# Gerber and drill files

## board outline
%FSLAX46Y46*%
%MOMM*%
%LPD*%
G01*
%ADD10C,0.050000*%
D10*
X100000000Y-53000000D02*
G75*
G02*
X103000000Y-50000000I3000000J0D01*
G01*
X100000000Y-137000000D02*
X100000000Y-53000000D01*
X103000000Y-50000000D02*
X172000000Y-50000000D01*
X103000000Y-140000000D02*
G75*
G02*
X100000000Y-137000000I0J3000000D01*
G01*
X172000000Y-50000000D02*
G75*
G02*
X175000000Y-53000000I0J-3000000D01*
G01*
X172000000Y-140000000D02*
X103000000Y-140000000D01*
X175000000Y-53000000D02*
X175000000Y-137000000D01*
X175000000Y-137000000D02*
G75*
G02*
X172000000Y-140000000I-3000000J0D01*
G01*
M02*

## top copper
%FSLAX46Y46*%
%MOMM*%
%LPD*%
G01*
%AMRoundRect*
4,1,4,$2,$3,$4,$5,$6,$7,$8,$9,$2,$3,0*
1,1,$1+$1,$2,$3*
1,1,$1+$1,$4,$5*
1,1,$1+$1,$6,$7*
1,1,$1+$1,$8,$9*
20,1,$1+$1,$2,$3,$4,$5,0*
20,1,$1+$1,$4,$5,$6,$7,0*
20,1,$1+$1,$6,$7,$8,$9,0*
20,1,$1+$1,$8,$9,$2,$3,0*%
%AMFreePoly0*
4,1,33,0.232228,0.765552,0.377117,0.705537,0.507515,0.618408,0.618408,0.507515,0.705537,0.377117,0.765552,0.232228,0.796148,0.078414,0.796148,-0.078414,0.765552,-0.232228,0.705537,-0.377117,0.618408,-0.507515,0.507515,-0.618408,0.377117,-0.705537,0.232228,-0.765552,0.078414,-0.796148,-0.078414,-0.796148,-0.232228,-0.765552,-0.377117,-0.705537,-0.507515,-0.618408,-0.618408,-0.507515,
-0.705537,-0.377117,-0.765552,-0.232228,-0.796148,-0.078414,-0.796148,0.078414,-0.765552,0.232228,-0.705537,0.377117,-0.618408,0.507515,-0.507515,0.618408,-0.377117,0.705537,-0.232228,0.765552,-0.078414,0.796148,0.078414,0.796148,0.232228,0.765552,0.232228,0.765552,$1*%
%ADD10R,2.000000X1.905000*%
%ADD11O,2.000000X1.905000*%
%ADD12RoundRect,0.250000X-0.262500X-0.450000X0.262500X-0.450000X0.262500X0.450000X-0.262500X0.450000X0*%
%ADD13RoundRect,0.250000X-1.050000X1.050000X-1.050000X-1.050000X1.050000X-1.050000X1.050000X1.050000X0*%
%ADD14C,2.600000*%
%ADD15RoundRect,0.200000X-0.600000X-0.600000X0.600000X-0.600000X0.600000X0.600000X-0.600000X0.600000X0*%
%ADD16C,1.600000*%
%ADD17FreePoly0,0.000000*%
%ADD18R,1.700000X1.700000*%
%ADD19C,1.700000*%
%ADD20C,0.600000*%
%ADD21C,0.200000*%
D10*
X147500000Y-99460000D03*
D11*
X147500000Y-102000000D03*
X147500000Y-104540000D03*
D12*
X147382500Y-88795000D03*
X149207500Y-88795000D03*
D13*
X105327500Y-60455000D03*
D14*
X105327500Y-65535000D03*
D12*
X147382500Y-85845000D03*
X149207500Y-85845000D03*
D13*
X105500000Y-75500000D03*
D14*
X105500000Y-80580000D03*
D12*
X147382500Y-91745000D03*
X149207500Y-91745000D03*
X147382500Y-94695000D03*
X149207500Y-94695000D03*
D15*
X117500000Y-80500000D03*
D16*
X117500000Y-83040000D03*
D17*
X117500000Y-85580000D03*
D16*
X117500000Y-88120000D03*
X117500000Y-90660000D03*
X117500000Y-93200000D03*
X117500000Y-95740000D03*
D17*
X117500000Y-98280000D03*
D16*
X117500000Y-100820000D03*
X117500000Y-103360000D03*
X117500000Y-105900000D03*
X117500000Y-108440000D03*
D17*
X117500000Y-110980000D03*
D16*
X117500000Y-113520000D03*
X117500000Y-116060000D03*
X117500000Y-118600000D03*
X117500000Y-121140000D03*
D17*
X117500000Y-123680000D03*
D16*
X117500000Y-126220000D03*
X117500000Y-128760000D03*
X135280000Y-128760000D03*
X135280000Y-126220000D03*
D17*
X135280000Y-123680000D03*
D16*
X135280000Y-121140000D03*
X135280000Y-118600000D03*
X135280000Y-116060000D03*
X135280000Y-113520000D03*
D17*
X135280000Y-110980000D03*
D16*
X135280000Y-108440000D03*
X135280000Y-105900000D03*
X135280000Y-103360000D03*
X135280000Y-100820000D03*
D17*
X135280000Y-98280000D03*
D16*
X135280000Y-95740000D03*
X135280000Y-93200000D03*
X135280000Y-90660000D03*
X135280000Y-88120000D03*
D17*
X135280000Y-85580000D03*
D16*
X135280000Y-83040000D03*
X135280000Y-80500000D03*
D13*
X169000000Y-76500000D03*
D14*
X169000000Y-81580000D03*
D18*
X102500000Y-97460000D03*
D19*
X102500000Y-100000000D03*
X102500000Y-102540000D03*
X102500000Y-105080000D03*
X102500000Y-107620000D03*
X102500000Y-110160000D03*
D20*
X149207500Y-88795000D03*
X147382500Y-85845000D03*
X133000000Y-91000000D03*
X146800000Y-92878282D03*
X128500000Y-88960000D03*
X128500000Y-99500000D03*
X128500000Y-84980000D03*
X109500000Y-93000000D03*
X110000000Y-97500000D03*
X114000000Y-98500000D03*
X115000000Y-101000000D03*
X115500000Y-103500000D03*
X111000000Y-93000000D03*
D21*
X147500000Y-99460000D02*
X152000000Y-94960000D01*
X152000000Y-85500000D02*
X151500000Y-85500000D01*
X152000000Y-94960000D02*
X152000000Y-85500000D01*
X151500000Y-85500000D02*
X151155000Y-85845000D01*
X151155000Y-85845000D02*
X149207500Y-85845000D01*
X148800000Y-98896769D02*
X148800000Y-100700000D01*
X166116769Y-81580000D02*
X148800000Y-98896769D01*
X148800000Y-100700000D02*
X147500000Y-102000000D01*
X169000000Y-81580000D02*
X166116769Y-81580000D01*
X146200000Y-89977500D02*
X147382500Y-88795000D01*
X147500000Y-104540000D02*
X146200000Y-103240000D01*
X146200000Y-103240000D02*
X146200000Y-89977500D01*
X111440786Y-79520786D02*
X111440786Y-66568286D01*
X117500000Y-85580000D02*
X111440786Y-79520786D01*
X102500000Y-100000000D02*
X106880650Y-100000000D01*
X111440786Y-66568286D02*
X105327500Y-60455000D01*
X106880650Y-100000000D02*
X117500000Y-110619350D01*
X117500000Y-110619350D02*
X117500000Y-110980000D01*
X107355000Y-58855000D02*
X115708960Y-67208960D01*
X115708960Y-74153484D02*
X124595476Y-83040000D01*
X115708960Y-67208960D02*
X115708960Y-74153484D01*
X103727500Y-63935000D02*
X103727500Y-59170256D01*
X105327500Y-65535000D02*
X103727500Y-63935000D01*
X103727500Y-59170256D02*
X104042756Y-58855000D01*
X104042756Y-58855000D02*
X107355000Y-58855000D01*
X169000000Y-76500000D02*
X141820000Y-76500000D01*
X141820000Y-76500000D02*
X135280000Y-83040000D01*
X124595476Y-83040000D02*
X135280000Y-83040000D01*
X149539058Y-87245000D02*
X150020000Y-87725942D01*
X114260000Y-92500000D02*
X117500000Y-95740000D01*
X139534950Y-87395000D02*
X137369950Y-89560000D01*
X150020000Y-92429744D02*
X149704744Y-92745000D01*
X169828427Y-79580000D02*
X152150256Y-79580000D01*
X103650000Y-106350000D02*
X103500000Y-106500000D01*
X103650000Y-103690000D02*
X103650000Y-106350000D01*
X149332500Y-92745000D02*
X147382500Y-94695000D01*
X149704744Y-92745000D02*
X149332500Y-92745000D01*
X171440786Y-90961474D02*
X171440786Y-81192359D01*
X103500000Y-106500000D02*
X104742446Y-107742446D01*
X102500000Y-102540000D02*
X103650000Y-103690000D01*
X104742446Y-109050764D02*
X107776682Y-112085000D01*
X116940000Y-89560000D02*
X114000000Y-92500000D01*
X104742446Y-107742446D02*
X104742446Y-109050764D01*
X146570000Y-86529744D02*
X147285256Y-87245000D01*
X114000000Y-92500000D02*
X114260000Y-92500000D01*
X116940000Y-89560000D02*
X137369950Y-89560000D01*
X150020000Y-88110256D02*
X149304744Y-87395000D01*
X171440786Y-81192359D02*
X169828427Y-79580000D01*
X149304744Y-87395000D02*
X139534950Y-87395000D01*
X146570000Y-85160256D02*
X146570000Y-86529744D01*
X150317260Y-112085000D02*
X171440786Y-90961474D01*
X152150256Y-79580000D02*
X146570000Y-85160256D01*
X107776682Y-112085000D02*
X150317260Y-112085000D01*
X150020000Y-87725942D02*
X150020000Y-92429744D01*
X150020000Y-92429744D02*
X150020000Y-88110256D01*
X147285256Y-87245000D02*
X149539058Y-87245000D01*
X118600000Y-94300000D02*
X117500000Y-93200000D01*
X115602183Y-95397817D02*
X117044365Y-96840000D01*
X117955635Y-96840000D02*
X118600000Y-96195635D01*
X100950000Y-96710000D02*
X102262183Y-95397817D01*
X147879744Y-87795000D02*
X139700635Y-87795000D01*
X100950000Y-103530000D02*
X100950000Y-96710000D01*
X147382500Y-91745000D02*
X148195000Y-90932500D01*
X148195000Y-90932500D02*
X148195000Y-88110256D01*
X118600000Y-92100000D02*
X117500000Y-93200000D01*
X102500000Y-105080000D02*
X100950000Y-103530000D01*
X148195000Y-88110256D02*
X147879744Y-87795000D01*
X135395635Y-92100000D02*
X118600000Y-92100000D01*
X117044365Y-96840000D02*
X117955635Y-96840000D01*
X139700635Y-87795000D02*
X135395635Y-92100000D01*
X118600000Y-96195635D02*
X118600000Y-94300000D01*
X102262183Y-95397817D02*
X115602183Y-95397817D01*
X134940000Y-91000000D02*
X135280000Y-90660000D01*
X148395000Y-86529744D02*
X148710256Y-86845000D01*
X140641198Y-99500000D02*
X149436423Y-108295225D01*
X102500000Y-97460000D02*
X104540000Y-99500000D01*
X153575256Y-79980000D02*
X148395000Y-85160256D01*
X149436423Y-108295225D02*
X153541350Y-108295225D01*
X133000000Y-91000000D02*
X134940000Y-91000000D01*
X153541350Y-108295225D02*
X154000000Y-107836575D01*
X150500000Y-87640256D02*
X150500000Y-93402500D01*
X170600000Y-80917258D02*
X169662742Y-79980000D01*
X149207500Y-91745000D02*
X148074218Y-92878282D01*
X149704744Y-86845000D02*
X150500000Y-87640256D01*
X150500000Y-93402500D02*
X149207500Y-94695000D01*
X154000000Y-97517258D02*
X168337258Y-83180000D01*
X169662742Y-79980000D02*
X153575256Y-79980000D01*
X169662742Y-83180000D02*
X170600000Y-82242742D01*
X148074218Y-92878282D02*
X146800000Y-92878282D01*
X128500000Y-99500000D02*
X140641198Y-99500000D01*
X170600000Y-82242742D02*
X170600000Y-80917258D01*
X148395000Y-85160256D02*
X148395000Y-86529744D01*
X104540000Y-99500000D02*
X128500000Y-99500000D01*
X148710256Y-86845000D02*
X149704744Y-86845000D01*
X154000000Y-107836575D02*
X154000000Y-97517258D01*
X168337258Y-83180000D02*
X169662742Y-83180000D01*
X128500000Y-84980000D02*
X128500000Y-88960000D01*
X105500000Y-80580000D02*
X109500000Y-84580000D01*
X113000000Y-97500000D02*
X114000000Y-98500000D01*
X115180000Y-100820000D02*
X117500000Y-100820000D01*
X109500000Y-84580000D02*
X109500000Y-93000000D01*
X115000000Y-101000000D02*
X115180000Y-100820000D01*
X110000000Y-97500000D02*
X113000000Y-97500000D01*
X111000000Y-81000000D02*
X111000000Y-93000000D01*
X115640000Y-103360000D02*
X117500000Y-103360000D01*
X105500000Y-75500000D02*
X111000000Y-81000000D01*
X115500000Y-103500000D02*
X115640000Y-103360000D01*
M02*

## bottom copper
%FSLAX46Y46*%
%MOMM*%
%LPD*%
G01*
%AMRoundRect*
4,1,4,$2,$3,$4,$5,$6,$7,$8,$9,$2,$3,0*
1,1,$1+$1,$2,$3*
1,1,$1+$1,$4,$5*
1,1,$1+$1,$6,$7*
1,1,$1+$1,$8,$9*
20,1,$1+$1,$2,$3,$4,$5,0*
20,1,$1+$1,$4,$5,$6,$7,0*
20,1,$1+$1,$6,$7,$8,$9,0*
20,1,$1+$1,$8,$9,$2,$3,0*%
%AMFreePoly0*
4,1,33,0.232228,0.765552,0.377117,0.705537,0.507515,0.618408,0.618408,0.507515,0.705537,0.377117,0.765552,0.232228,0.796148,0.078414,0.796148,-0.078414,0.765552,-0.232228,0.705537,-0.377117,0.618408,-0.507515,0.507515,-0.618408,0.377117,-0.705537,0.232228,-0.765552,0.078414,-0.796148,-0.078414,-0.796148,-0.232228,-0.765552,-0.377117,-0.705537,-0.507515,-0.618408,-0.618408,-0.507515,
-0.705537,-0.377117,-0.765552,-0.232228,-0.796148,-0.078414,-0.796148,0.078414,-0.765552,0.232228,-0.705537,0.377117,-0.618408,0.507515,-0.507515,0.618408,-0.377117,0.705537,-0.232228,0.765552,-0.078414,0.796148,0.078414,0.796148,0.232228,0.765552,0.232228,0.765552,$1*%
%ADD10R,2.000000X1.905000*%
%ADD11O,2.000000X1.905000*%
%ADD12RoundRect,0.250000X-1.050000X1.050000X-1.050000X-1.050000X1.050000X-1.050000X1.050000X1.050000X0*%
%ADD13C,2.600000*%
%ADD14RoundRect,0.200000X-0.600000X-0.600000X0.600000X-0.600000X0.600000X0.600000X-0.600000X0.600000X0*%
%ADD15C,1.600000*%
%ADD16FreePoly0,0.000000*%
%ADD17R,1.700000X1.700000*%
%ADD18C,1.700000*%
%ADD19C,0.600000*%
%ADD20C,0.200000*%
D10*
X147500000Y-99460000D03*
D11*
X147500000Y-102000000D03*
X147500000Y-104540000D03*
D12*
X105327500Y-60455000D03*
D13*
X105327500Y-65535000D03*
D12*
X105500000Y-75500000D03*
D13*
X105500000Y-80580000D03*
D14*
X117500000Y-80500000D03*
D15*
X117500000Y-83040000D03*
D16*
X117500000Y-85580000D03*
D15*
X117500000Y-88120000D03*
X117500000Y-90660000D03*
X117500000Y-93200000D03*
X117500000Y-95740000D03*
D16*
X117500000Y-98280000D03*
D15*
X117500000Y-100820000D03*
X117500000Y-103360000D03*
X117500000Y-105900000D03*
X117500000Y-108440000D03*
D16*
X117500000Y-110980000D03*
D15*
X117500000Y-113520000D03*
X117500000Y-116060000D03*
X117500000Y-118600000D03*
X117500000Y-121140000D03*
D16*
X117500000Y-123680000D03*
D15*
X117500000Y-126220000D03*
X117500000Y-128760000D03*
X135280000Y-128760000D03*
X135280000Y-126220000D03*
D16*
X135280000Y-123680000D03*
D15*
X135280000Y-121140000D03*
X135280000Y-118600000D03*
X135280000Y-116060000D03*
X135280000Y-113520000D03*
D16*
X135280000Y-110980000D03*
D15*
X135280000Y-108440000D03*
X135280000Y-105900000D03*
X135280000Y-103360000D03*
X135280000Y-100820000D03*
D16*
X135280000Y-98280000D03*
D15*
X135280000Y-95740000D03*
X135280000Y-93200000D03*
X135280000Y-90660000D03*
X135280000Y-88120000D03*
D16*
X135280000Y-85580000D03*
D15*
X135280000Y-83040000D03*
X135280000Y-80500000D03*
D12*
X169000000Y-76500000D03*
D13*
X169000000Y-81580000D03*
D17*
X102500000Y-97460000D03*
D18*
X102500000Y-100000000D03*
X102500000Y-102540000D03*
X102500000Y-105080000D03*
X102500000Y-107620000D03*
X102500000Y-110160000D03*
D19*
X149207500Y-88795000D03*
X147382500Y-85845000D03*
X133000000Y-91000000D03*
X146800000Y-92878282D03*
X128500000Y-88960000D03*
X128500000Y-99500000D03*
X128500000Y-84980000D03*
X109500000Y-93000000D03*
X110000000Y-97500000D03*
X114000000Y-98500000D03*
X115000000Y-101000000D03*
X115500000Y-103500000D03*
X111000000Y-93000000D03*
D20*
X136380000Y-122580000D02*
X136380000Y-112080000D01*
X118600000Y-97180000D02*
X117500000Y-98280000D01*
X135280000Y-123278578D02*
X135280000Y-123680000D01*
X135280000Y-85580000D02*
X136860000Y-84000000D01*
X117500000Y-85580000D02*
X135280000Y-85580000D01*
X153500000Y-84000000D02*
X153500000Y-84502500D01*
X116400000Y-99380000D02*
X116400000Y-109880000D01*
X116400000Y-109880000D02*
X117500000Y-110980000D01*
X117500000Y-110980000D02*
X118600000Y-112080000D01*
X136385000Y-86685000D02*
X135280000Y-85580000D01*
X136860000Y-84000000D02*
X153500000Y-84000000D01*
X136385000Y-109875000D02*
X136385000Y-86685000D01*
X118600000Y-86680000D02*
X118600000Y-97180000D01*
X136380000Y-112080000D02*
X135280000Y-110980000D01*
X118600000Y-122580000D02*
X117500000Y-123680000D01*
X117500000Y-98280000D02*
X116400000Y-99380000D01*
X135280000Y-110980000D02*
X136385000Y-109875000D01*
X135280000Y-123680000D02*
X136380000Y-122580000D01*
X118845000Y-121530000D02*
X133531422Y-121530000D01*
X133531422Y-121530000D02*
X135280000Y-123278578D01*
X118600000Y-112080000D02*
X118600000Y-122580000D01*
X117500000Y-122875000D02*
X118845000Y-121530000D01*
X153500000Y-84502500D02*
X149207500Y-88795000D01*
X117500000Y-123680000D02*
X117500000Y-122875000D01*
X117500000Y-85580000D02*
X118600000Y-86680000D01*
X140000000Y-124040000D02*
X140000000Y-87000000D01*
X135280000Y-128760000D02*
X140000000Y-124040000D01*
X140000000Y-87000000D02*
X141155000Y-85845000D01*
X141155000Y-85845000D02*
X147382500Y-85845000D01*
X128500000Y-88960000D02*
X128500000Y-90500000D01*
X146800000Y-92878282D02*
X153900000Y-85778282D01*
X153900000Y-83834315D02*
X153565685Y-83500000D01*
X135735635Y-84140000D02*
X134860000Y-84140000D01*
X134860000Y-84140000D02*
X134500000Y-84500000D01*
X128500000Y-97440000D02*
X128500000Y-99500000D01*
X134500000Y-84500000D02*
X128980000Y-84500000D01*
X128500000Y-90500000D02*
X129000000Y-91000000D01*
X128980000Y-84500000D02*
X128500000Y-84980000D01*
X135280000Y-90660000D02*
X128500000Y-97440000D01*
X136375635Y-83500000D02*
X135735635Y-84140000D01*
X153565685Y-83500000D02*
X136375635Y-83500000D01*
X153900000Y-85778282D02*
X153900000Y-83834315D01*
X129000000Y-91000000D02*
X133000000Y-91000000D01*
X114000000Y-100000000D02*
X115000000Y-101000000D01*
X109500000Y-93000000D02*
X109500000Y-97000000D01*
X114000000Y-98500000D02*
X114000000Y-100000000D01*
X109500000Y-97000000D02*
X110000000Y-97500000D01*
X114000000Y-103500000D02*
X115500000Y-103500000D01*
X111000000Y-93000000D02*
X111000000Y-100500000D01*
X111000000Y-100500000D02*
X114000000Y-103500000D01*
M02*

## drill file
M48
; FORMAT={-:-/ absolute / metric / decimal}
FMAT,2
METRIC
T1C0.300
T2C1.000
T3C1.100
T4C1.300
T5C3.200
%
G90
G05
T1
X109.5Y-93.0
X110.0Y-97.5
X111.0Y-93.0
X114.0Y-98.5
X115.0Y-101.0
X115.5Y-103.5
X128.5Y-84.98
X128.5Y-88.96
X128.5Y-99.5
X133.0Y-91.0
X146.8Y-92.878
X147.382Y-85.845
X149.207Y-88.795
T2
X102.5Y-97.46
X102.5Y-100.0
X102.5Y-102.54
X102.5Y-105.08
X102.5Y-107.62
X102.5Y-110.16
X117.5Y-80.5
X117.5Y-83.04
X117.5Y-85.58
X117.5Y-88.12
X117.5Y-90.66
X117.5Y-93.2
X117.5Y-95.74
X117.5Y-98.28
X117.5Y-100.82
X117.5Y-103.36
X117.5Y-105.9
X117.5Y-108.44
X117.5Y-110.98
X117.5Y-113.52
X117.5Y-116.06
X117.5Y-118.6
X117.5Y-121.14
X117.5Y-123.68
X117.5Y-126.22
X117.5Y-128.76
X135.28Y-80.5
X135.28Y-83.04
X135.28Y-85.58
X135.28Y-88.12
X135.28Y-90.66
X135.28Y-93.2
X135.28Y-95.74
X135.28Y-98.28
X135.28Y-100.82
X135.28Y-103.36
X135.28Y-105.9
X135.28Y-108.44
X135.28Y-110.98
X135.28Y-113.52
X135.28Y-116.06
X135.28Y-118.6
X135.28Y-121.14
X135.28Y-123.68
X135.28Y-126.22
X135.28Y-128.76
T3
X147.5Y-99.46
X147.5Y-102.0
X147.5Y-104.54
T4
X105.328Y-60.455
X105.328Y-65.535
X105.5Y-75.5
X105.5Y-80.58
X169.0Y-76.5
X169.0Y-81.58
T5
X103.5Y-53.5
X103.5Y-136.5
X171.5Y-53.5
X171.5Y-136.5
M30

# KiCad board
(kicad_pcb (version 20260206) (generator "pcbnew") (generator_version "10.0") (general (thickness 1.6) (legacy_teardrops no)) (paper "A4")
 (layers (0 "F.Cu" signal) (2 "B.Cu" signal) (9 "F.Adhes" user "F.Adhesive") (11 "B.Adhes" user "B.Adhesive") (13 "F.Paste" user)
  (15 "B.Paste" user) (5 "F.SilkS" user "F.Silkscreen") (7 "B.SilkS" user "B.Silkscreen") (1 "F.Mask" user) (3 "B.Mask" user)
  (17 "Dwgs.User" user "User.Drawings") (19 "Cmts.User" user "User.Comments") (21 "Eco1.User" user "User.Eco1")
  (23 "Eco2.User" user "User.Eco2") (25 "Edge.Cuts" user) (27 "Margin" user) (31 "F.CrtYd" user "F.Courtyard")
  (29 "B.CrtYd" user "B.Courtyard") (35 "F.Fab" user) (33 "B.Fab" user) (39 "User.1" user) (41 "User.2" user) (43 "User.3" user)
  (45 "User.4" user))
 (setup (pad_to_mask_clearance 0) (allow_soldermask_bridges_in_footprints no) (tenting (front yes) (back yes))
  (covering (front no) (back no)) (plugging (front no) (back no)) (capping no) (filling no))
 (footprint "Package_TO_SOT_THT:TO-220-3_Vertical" (layer "F.Cu") (at 147.5 99.46 -90)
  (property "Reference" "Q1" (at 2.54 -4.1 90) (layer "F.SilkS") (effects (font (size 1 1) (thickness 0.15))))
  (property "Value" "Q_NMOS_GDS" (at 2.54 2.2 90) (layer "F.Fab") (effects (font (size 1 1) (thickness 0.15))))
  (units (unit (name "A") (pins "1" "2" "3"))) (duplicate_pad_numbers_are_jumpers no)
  (pad "1" thru_hole rect (at 0 0 270) (size 1.905 2) (drill 1.1) (layers "*.Cu" "*.Mask") (remove_unused_layers no) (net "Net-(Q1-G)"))
  (pad "2" thru_hole oval (at 2.54 0 270) (size 1.905 2) (drill 1.1) (layers "*.Cu" "*.Mask") (remove_unused_layers no)
   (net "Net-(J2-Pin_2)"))
  (pad "3" thru_hole oval (at 5.08 0 270) (size 1.905 2) (drill 1.1) (layers "*.Cu" "*.Mask") (remove_unused_layers no) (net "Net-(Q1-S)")))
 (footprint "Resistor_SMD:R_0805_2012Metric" (layer "F.Cu") (at 148.295 88.795)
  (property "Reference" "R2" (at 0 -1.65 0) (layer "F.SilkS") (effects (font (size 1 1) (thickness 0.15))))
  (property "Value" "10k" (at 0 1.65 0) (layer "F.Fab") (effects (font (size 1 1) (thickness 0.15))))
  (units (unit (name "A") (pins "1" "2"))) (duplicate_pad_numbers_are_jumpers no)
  (pad "1" smd roundrect (at -0.9125 0) (size 1.025 1.4) (layers "F.Cu" "F.Mask" "F.Paste") (roundrect_rratio 0.243902) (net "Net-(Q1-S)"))
  (pad "2" smd roundrect (at 0.9125 0) (size 1.025 1.4) (layers "F.Cu" "F.Mask" "F.Paste") (roundrect_rratio 0.243902) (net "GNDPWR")))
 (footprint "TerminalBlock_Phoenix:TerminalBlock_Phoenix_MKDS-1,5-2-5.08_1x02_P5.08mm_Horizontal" (layer "F.Cu") (at 105.3275 60.455 -90)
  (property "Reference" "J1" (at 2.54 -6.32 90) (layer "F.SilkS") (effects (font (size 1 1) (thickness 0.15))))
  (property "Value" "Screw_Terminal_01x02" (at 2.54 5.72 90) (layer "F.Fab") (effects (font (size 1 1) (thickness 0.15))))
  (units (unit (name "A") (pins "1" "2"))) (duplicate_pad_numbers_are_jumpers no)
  (pad "1" thru_hole roundrect (at 0 0 270) (size 2.6 2.6) (drill 1.3) (layers "*.Cu" "*.Mask") (remove_unused_layers no)
   (roundrect_rratio 0.096154) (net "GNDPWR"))
  (pad "2" thru_hole circle (at 5.08 0 270) (size 2.6 2.6) (drill 1.3) (layers "*.Cu" "*.Mask") (remove_unused_layers no)
   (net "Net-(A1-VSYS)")))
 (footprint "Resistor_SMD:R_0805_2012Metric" (layer "F.Cu") (at 148.295 85.845)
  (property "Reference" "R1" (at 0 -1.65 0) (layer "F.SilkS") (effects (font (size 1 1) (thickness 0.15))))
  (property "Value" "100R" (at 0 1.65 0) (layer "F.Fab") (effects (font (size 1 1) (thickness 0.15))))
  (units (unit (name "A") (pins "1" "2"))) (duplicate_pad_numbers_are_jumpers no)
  (pad "1" smd roundrect (at -0.9125 0) (size 1.025 1.4) (layers "F.Cu" "F.Mask" "F.Paste") (roundrect_rratio 0.243902)
   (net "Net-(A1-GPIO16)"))
  (pad "2" smd roundrect (at 0.9125 0) (size 1.025 1.4) (layers "F.Cu" "F.Mask" "F.Paste") (roundrect_rratio 0.243902) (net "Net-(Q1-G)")))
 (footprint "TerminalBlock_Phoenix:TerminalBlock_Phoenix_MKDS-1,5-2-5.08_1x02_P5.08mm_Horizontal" (layer "F.Cu") (at 105.5 75.5 -90)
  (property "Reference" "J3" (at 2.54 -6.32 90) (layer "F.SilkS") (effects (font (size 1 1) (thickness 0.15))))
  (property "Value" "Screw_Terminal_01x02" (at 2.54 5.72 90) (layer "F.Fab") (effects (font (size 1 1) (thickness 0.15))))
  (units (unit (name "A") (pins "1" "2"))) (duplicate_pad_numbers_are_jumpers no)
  (pad "1" thru_hole roundrect (at 0 0 270) (size 2.6 2.6) (drill 1.3) (layers "*.Cu" "*.Mask") (remove_unused_layers no)
   (roundrect_rratio 0.096154) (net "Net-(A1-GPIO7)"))
  (pad "2" thru_hole circle (at 5.08 0 270) (size 2.6 2.6) (drill 1.3) (layers "*.Cu" "*.Mask") (remove_unused_layers no)
   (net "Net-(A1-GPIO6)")))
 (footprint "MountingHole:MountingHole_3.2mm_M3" (layer "F.Cu") (at 171.5 53.5)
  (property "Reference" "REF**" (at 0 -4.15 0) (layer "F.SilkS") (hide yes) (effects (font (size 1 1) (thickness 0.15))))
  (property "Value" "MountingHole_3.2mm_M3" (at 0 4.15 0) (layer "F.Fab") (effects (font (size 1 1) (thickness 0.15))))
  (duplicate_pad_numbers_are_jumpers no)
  (pad "" np_thru_hole circle (at 0 0) (size 3.2 3.2) (drill 3.2) (layers "*.Cu" "*.Mask")))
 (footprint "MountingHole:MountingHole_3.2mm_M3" (layer "F.Cu") (at 103.5 136.5)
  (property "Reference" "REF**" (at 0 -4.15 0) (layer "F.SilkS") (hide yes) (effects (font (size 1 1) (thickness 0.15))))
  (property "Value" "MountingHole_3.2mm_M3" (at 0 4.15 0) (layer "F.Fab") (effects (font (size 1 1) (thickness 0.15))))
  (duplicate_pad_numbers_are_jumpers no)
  (pad "" np_thru_hole circle (at 0 0) (size 3.2 3.2) (drill 3.2) (layers "*.Cu" "*.Mask")))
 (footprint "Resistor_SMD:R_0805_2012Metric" (layer "F.Cu") (at 148.295 91.745)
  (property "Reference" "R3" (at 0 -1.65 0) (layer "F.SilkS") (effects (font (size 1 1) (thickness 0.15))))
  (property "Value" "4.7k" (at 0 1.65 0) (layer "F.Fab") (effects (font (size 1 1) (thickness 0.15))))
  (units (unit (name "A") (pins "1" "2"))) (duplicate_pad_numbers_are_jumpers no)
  (pad "1" smd roundrect (at -0.9125 0) (size 1.025 1.4) (layers "F.Cu" "F.Mask" "F.Paste") (roundrect_rratio 0.243902)
   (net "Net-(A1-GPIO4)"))
  (pad "2" smd roundrect (at 0.9125 0) (size 1.025 1.4) (layers "F.Cu" "F.Mask" "F.Paste") (roundrect_rratio 0.243902) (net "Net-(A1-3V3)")))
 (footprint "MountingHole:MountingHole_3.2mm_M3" (layer "F.Cu") (at 171.5 136.5)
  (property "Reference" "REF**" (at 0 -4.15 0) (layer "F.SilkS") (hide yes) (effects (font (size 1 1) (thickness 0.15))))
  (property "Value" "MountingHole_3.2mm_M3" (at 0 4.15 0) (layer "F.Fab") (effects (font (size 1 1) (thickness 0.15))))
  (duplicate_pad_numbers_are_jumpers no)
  (pad "" np_thru_hole circle (at 0 0) (size 3.2 3.2) (drill 3.2) (layers "*.Cu" "*.Mask")))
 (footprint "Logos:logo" (layer "F.Cu") (at 158.5 120)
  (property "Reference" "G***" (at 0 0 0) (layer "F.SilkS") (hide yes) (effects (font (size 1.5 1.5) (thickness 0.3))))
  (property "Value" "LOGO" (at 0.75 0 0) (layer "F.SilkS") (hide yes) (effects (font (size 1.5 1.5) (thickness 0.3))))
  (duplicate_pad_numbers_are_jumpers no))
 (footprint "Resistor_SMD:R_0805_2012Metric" (layer "F.Cu") (at 148.295 94.695)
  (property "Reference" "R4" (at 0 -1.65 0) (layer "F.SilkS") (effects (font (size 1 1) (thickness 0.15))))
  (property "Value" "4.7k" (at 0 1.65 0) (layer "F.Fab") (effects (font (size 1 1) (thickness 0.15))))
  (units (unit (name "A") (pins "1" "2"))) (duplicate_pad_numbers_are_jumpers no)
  (pad "1" smd roundrect (at -0.9125 0) (size 1.025 1.4) (layers "F.Cu" "F.Mask" "F.Paste") (roundrect_rratio 0.243902)
   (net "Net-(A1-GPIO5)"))
  (pad "2" smd roundrect (at 0.9125 0) (size 1.025 1.4) (layers "F.Cu" "F.Mask" "F.Paste") (roundrect_rratio 0.243902) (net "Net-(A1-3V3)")))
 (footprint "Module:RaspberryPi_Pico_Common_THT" (layer "F.Cu") (at 117.5 80.5)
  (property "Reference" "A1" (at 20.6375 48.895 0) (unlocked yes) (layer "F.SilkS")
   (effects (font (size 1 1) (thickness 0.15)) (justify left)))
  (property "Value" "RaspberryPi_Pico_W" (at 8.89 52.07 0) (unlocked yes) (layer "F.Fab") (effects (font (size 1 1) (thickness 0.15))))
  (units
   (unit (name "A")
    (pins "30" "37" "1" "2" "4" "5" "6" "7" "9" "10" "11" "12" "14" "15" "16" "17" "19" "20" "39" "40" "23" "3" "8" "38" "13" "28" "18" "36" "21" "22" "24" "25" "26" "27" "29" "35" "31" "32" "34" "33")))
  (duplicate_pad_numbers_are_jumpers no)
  (pad "1" thru_hole roundrect (at 0 0) (size 1.6 1.6) (drill 1) (layers "*.Cu" "*.Mask") (remove_unused_layers no) (roundrect_rratio 0.125)
   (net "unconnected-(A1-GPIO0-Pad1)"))
  (pad "2" thru_hole circle (at 0 2.54) (size 1.6 1.6) (drill 1) (layers "*.Cu" "*.Mask") (remove_unused_layers no)
   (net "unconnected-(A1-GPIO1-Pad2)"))
  (pad "3" thru_hole custom (at 0 5.08) (size 1.6 1.6) (drill 1) (layers "*.Cu" "*.Mask") (remove_unused_layers no) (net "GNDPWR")
   (options (clearance outline) (anchor circle)) (primitives))
  (pad "4" thru_hole circle (at 0 7.62) (size 1.6 1.6) (drill 1) (layers "*.Cu" "*.Mask") (remove_unused_layers no)
   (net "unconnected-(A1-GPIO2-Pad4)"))
  (pad "5" thru_hole circle (at 0 10.16) (size 1.6 1.6) (drill 1) (layers "*.Cu" "*.Mask") (remove_unused_layers no)
   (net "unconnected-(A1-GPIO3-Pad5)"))
  (pad "6" thru_hole circle (at 0 12.7) (size 1.6 1.6) (drill 1) (layers "*.Cu" "*.Mask") (remove_unused_layers no) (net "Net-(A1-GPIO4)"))
  (pad "7" thru_hole circle (at 0 15.24) (size 1.6 1.6) (drill 1) (layers "*.Cu" "*.Mask") (remove_unused_layers no) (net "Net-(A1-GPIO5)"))
  (pad "8" thru_hole custom (at 0 17.78) (size 1.6 1.6) (drill 1) (layers "*.Cu" "*.Mask") (remove_unused_layers no) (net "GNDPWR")
   (options (clearance outline) (anchor circle)) (primitives))
  (pad "9" thru_hole circle (at 0 20.32) (size 1.6 1.6) (drill 1) (layers "*.Cu" "*.Mask") (remove_unused_layers no) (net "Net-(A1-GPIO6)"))
  (pad "10" thru_hole circle (at 0 22.86) (size 1.6 1.6) (drill 1) (layers "*.Cu" "*.Mask") (remove_unused_layers no) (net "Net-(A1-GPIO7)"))
  (pad "11" thru_hole circle (at 0 25.4) (size 1.6 1.6) (drill 1) (layers "*.Cu" "*.Mask") (remove_unused_layers no)
   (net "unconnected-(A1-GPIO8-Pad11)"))
  (pad "12" thru_hole circle (at 0 27.94) (size 1.6 1.6) (drill 1) (layers "*.Cu" "*.Mask") (remove_unused_layers no)
   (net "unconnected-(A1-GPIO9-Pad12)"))
  (pad "13" thru_hole custom (at 0 30.48) (size 1.6 1.6) (drill 1) (layers "*.Cu" "*.Mask") (remove_unused_layers no) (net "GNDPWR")
   (options (clearance outline) (anchor circle)) (primitives))
  (pad "14" thru_hole circle (at 0 33.02) (size 1.6 1.6) (drill 1) (layers "*.Cu" "*.Mask") (remove_unused_layers no)
   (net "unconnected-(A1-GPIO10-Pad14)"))
  (pad "15" thru_hole circle (at 0 35.56) (size 1.6 1.6) (drill 1) (layers "*.Cu" "*.Mask") (remove_unused_layers no)
   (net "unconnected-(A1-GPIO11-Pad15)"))
  (pad "16" thru_hole circle (at 0 38.1) (size 1.6 1.6) (drill 1) (layers "*.Cu" "*.Mask") (remove_unused_layers no)
   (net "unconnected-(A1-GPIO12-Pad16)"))
  (pad "17" thru_hole circle (at 0 40.64) (size 1.6 1.6) (drill 1) (layers "*.Cu" "*.Mask") (remove_unused_layers no)
   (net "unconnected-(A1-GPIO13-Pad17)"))
  (pad "18" thru_hole custom (at 0 43.18) (size 1.6 1.6) (drill 1) (layers "*.Cu" "*.Mask") (remove_unused_layers no) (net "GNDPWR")
   (options (clearance outline) (anchor circle)) (primitives))
  (pad "19" thru_hole circle (at 0 45.72) (size 1.6 1.6) (drill 1) (layers "*.Cu" "*.Mask") (remove_unused_layers no)
   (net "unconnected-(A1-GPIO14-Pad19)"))
  (pad "20" thru_hole circle (at 0 48.26) (size 1.6 1.6) (drill 1) (layers "*.Cu" "*.Mask") (remove_unused_layers no)
   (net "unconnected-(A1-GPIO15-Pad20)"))
  (pad "21" thru_hole circle (at 17.78 48.26) (size 1.6 1.6) (drill 1) (layers "*.Cu" "*.Mask") (remove_unused_layers no)
   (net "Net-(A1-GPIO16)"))
  (pad "22" thru_hole circle (at 17.78 45.72) (size 1.6 1.6) (drill 1) (layers "*.Cu" "*.Mask") (remove_unused_layers no)
   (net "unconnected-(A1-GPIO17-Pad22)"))
  (pad "23" thru_hole custom (at 17.78 43.18) (size 1.6 1.6) (drill 1) (layers "*.Cu" "*.Mask") (remove_unused_layers no) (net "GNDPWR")
   (options (clearance outline) (anchor circle)) (primitives))
  (pad "24" thru_hole circle (at 17.78 40.64) (size 1.6 1.6) (drill 1) (layers "*.Cu" "*.Mask") (remove_unused_layers no)
   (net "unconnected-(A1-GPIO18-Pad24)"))
  (pad "25" thru_hole circle (at 17.78 38.1) (size 1.6 1.6) (drill 1) (layers "*.Cu" "*.Mask") (remove_unused_layers no)
   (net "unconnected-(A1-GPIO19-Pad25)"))
  (pad "26" thru_hole circle (at 17.78 35.56) (size 1.6 1.6) (drill 1) (layers "*.Cu" "*.Mask") (remove_unused_layers no)
   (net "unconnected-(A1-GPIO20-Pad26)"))
  (pad "27" thru_hole circle (at 17.78 33.02) (size 1.6 1.6) (drill 1) (layers "*.Cu" "*.Mask") (remove_unused_layers no)
   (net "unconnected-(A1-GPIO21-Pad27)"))
  (pad "28" thru_hole custom (at 17.78 30.48) (size 1.6 1.6) (drill 1) (layers "*.Cu" "*.Mask") (remove_unused_layers no) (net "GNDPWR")
   (options (clearance outline) (anchor circle)) (primitives))
  (pad "29" thru_hole circle (at 17.78 27.94) (size 1.6 1.6) (drill 1) (layers "*.Cu" "*.Mask") (remove_unused_layers no)
   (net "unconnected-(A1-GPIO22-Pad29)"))
  (pad "30" thru_hole circle (at 17.78 25.4) (size 1.6 1.6) (drill 1) (layers "*.Cu" "*.Mask") (remove_unused_layers no)
   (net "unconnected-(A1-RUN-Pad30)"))
  (pad "31" thru_hole circle (at 17.78 22.86) (size 1.6 1.6) (drill 1) (layers "*.Cu" "*.Mask") (remove_unused_layers no)
   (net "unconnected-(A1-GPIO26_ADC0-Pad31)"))
  (pad "32" thru_hole circle (at 17.78 20.32) (size 1.6 1.6) (drill 1) (layers "*.Cu" "*.Mask") (remove_unused_layers no)
   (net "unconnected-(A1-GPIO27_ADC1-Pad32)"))
  (pad "33" thru_hole custom (at 17.78 17.78) (size 1.6 1.6) (drill 1) (layers "*.Cu" "*.Mask") (remove_unused_layers no)
   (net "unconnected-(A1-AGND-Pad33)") (options (clearance outline) (anchor circle)) (primitives))
  (pad "34" thru_hole circle (at 17.78 15.24) (size 1.6 1.6) (drill 1) (layers "*.Cu" "*.Mask") (remove_unused_layers no)
   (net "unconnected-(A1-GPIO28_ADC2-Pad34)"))
  (pad "35" thru_hole circle (at 17.78 12.7) (size 1.6 1.6) (drill 1) (layers "*.Cu" "*.Mask") (remove_unused_layers no)
   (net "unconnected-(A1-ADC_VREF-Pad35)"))
  (pad "36" thru_hole circle (at 17.78 10.16) (size 1.6 1.6) (drill 1) (layers "*.Cu" "*.Mask") (remove_unused_layers no)
   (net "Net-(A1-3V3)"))
  (pad "37" thru_hole circle (at 17.78 7.62) (size 1.6 1.6) (drill 1) (layers "*.Cu" "*.Mask") (remove_unused_layers no)
   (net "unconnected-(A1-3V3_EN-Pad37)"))
  (pad "38" thru_hole custom (at 17.78 5.08) (size 1.6 1.6) (drill 1) (layers "*.Cu" "*.Mask") (remove_unused_layers no) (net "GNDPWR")
   (options (clearance outline) (anchor circle)) (primitives))
  (pad "39" thru_hole circle (at 17.78 2.54) (size 1.6 1.6) (drill 1) (layers "*.Cu" "*.Mask") (remove_unused_layers no)
   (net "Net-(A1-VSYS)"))
  (pad "40" thru_hole circle (at 17.78 0) (size 1.6 1.6) (drill 1) (layers "*.Cu" "*.Mask") (remove_unused_layers no)
   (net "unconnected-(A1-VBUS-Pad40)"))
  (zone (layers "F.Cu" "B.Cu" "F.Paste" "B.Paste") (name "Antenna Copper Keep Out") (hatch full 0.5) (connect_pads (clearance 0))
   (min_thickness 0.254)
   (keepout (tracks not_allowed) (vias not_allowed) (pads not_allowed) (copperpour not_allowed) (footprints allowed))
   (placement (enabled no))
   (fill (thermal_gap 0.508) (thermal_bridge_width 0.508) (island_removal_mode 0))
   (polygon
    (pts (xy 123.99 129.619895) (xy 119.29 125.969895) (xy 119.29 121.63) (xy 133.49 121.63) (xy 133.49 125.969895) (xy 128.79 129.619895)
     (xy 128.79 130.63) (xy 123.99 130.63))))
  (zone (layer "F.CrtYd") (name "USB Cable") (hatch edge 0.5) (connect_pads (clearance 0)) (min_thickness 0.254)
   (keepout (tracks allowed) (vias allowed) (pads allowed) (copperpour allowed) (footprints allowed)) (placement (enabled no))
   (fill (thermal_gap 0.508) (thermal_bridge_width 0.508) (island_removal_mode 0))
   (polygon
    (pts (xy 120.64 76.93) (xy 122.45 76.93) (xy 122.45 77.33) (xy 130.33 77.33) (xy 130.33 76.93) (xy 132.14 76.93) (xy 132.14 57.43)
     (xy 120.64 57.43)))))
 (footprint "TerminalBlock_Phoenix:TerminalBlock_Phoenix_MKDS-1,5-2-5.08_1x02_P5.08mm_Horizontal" (layer "F.Cu") (at 169 76.5 -90)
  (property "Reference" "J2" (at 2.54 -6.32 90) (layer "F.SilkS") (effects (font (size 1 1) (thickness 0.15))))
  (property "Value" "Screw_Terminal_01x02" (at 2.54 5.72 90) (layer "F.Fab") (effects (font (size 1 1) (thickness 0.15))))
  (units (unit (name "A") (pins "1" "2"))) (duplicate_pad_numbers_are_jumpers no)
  (pad "1" thru_hole roundrect (at 0 0 270) (size 2.6 2.6) (drill 1.3) (layers "*.Cu" "*.Mask") (remove_unused_layers no)
   (roundrect_rratio 0.096154) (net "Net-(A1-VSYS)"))
  (pad "2" thru_hole circle (at 5.08 0 270) (size 2.6 2.6) (drill 1.3) (layers "*.Cu" "*.Mask") (remove_unused_layers no)
   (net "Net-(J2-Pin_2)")))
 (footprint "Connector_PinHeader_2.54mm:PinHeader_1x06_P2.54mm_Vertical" (layer "F.Cu") (at 102.5 97.46)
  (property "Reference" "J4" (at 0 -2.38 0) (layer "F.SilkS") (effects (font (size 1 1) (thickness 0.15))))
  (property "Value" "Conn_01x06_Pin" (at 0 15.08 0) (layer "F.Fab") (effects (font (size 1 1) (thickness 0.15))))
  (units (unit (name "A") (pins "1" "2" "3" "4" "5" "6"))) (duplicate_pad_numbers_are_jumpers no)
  (pad "1" thru_hole rect (at 0 0) (size 1.7 1.7) (drill 1) (layers "*.Cu" "*.Mask") (remove_unused_layers no) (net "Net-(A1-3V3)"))
  (pad "2" thru_hole circle (at 0 2.54) (size 1.7 1.7) (drill 1) (layers "*.Cu" "*.Mask") (remove_unused_layers no) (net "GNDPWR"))
  (pad "3" thru_hole circle (at 0 5.08) (size 1.7 1.7) (drill 1) (layers "*.Cu" "*.Mask") (remove_unused_layers no) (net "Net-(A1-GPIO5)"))
  (pad "4" thru_hole circle (at 0 7.62) (size 1.7 1.7) (drill 1) (layers "*.Cu" "*.Mask") (remove_unused_layers no) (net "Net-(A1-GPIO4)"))
  (pad "5" thru_hole circle (at 0 10.16) (size 1.7 1.7) (drill 1) (layers "*.Cu" "*.Mask") (remove_unused_layers no)
   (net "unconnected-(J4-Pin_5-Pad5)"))
  (pad "6" thru_hole circle (at 0 12.7) (size 1.7 1.7) (drill 1) (layers "*.Cu" "*.Mask") (remove_unused_layers no)
   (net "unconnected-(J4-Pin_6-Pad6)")))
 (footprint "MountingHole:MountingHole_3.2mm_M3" (layer "F.Cu") (at 103.5 53.5)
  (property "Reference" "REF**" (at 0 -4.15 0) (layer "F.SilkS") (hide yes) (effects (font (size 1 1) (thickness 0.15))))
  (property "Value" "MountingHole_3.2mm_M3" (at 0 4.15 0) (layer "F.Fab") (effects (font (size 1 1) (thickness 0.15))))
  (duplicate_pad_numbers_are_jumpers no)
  (pad "" np_thru_hole circle (at 0 0) (size 3.2 3.2) (drill 3.2) (layers "*.Cu" "*.Mask")))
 (gr_arc (start 100 53) (mid 100.87868 50.87868) (end 103 50) (stroke (width 0.05) (type default)) (layer "Edge.Cuts"))
 (gr_line (start 100 137) (end 100 53) (stroke (width 0.05) (type default)) (layer "Edge.Cuts"))
 (gr_line (start 103 50) (end 172 50) (stroke (width 0.05) (type default)) (layer "Edge.Cuts"))
 (gr_arc (start 103 140) (mid 100.87868 139.12132) (end 100 137) (stroke (width 0.05) (type default)) (layer "Edge.Cuts"))
 (gr_arc (start 172 50) (mid 174.12132 50.87868) (end 175 53) (stroke (width 0.05) (type default)) (layer "Edge.Cuts"))
 (gr_line (start 172 140) (end 103 140) (stroke (width 0.05) (type default)) (layer "Edge.Cuts"))
 (gr_line (start 175 53) (end 175 137) (stroke (width 0.05) (type default)) (layer "Edge.Cuts"))
 (gr_arc (start 175 137) (mid 174.12132 139.12132) (end 172 140) (stroke (width 0.05) (type default)) (layer "Edge.Cuts"))
 (segment (start 147.5 99.46) (end 152 94.96) (width 0.2) (layer "F.Cu") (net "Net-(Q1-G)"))
 (segment (start 152 85.5) (end 151.5 85.5) (width 0.2) (layer "F.Cu") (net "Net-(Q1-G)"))
 (segment (start 152 94.96) (end 152 85.5) (width 0.2) (layer "F.Cu") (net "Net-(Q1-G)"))
 (segment (start 151.5 85.5) (end 151.155 85.845) (width 0.2) (layer "F.Cu") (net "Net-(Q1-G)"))
 (segment (start 151.155 85.845) (end 149.2075 85.845) (width 0.2) (layer "F.Cu") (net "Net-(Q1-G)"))
 (segment (start 148.8 98.896769) (end 148.8 100.7) (width 0.2) (layer "F.Cu") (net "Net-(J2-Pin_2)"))
 (segment (start 166.116769 81.58) (end 148.8 98.896769) (width 0.2) (layer "F.Cu") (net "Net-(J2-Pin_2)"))
 (segment (start 148.8 100.7) (end 147.5 102) (width 0.2) (layer "F.Cu") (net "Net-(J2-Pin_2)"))
 (segment (start 169 81.58) (end 166.116769 81.58) (width 0.2) (layer "F.Cu") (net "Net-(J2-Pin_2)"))
 (segment (start 146.2 89.9775) (end 147.3825 88.795) (width 0.2) (layer "F.Cu") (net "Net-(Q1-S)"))
 (segment (start 147.5 104.54) (end 146.2 103.24) (width 0.2) (layer "F.Cu") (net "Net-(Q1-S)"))
 (segment (start 146.2 103.24) (end 146.2 89.9775) (width 0.2) (layer "F.Cu") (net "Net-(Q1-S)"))
 (segment (start 111.440786 79.520786) (end 111.440786 66.568286) (width 0.2) (layer "F.Cu") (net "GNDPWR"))
 (segment (start 117.5 85.58) (end 111.440786 79.520786) (width 0.2) (layer "F.Cu") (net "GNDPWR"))
 (segment (start 102.5 100) (end 106.88065 100) (width 0.2) (layer "F.Cu") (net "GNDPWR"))
 (segment (start 111.440786 66.568286) (end 105.3275 60.455) (width 0.2) (layer "F.Cu") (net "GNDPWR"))
 (segment (start 106.88065 100) (end 117.5 110.61935) (width 0.2) (layer "F.Cu") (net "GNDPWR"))
 (segment (start 117.5 110.61935) (end 117.5 110.98) (width 0.2) (layer "F.Cu") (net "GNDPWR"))
 (via (at 149.2075 88.795) (size 0.6) (drill 0.3) (layers "F.Cu" "B.Cu") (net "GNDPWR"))
 (segment (start 136.38 122.58) (end 136.38 112.08) (width 0.2) (layer "B.Cu") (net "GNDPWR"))
 (segment (start 118.6 97.18) (end 117.5 98.28) (width 0.2) (layer "B.Cu") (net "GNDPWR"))
 (segment (start 135.28 123.278578) (end 135.28 123.68) (width 0.2) (layer "B.Cu") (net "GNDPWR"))
 (segment (start 135.28 85.58) (end 136.86 84) (width 0.2) (layer "B.Cu") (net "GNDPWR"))
 (segment (start 117.5 85.58) (end 135.28 85.58) (width 0.2) (layer "B.Cu") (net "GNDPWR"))
 (segment (start 153.5 84) (end 153.5 84.5025) (width 0.2) (layer "B.Cu") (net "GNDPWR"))
 (segment (start 116.4 99.38) (end 116.4 109.88) (width 0.2) (layer "B.Cu") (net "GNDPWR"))
 (segment (start 116.4 109.88) (end 117.5 110.98) (width 0.2) (layer "B.Cu") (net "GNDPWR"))
 (segment (start 117.5 110.98) (end 118.6 112.08) (width 0.2) (layer "B.Cu") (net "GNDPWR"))
 (segment (start 136.385 86.685) (end 135.28 85.58) (width 0.2) (layer "B.Cu") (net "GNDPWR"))
 (segment (start 136.86 84) (end 153.5 84) (width 0.2) (layer "B.Cu") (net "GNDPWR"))
 (segment (start 136.385 109.875) (end 136.385 86.685) (width 0.2) (layer "B.Cu") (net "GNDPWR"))
 (segment (start 118.6 86.68) (end 118.6 97.18) (width 0.2) (layer "B.Cu") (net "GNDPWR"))
 (segment (start 136.38 112.08) (end 135.28 110.98) (width 0.2) (layer "B.Cu") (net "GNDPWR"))
 (segment (start 118.6 122.58) (end 117.5 123.68) (width 0.2) (layer "B.Cu") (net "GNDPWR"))
 (segment (start 117.5 98.28) (end 116.4 99.38) (width 0.2) (layer "B.Cu") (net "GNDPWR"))
 (segment (start 135.28 110.98) (end 136.385 109.875) (width 0.2) (layer "B.Cu") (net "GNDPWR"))
 (segment (start 135.28 123.68) (end 136.38 122.58) (width 0.2) (layer "B.Cu") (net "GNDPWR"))
 (segment (start 118.845 121.53) (end 133.531422 121.53) (width 0.2) (layer "B.Cu") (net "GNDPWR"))
 (segment (start 133.531422 121.53) (end 135.28 123.278578) (width 0.2) (layer "B.Cu") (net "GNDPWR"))
 (segment (start 118.6 112.08) (end 118.6 122.58) (width 0.2) (layer "B.Cu") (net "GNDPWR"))
 (segment (start 117.5 122.875) (end 118.845 121.53) (width 0.2) (layer "B.Cu") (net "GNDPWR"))
 (segment (start 153.5 84.5025) (end 149.2075 88.795) (width 0.2) (layer "B.Cu") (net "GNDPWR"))
 (segment (start 117.5 123.68) (end 117.5 122.875) (width 0.2) (layer "B.Cu") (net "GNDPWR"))
 (segment (start 117.5 85.58) (end 118.6 86.68) (width 0.2) (layer "B.Cu") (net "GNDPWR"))
 (segment (start 107.355 58.855) (end 115.70896 67.20896) (width 0.2) (layer "F.Cu") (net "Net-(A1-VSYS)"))
 (segment (start 115.70896 74.153484) (end 124.595476 83.04) (width 0.2) (layer "F.Cu") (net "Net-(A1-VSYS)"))
 (segment (start 115.70896 67.20896) (end 115.70896 74.153484) (width 0.2) (layer "F.Cu") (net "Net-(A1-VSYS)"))
 (segment (start 103.7275 63.935) (end 103.7275 59.170256) (width 0.2) (layer "F.Cu") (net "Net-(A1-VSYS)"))
 (segment (start 105.3275 65.535) (end 103.7275 63.935) (width 0.2) (layer "F.Cu") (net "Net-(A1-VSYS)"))
 (segment (start 103.7275 59.170256) (end 104.042756 58.855) (width 0.2) (layer "F.Cu") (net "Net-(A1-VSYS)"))
 (segment (start 104.042756 58.855) (end 107.355 58.855) (width 0.2) (layer "F.Cu") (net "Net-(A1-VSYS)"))
 (segment (start 169 76.5) (end 141.82 76.5) (width 0.2) (layer "F.Cu") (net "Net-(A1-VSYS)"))
 (segment (start 141.82 76.5) (end 135.28 83.04) (width 0.2) (layer "F.Cu") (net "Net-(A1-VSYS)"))
 (segment (start 124.595476 83.04) (end 135.28 83.04) (width 0.2) (layer "F.Cu") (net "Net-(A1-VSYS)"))
 (via (at 147.3825 85.845) (size 0.6) (drill 0.3) (layers "F.Cu" "B.Cu") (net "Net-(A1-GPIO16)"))
 (segment (start 140 124.04) (end 140 87) (width 0.2) (layer "B.Cu") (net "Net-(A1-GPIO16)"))
 (segment (start 135.28 128.76) (end 140 124.04) (width 0.2) (layer "B.Cu") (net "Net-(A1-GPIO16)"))
 (segment (start 140 87) (end 141.155 85.845) (width 0.2) (layer "B.Cu") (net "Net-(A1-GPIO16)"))
 (segment (start 141.155 85.845) (end 147.3825 85.845) (width 0.2) (layer "B.Cu") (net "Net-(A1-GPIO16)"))
 (segment (start 149.539058 87.245) (end 150.02 87.725942) (width 0.2) (layer "F.Cu") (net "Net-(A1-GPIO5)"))
 (segment (start 114.26 92.5) (end 117.5 95.74) (width 0.2) (layer "F.Cu") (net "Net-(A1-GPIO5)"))
 (segment (start 139.53495 87.395) (end 137.36995 89.56) (width 0.2) (layer "F.Cu") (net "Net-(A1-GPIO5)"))
 (segment (start 150.02 92.429744) (end 149.704744 92.745) (width 0.2) (layer "F.Cu") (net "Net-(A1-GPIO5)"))
 (segment (start 169.828427 79.58) (end 152.150256 79.58) (width 0.2) (layer "F.Cu") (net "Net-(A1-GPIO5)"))
 (segment (start 103.65 106.35) (end 103.5 106.5) (width 0.2) (layer "F.Cu") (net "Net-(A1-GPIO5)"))
 (segment (start 103.65 103.69) (end 103.65 106.35) (width 0.2) (layer "F.Cu") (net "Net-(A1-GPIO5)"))
 (segment (start 149.3325 92.745) (end 147.3825 94.695) (width 0.2) (layer "F.Cu") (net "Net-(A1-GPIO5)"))
 (segment (start 149.704744 92.745) (end 149.3325 92.745) (width 0.2) (layer "F.Cu") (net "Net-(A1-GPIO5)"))
 (segment (start 171.440786 90.961474) (end 171.440786 81.192359) (width 0.2) (layer "F.Cu") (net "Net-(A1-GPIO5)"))
 (segment (start 103.5 106.5) (end 104.742446 107.742446) (width 0.2) (layer "F.Cu") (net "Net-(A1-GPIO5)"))
 (segment (start 102.5 102.54) (end 103.65 103.69) (width 0.2) (layer "F.Cu") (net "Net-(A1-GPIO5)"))
 (segment (start 104.742446 109.050764) (end 107.776682 112.085) (width 0.2) (layer "F.Cu") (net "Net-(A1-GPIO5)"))
 (segment (start 116.94 89.56) (end 114 92.5) (width 0.2) (layer "F.Cu") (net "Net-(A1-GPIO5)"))
 (segment (start 104.742446 107.742446) (end 104.742446 109.050764) (width 0.2) (layer "F.Cu") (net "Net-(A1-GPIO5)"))
 (segment (start 146.57 86.529744) (end 147.285256 87.245) (width 0.2) (layer "F.Cu") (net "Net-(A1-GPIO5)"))
 (segment (start 114 92.5) (end 114.26 92.5) (width 0.2) (layer "F.Cu") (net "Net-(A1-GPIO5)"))
 (segment (start 116.94 89.56) (end 137.36995 89.56) (width 0.2) (layer "F.Cu") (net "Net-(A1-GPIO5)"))
 (segment (start 150.02 88.110256) (end 149.304744 87.395) (width 0.2) (layer "F.Cu") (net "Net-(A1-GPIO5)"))
 (segment (start 171.440786 81.192359) (end 169.828427 79.58) (width 0.2) (layer "F.Cu") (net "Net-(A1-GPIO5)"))
 (segment (start 149.304744 87.395) (end 139.53495 87.395) (width 0.2) (layer "F.Cu") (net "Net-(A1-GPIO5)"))
 (segment (start 146.57 85.160256) (end 146.57 86.529744) (width 0.2) (layer "F.Cu") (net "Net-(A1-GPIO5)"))
 (segment (start 150.31726 112.085) (end 171.440786 90.961474) (width 0.2) (layer "F.Cu") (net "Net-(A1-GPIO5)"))
 (segment (start 152.150256 79.58) (end 146.57 85.160256) (width 0.2) (layer "F.Cu") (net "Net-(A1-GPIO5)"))
 (segment (start 107.776682 112.085) (end 150.31726 112.085) (width 0.2) (layer "F.Cu") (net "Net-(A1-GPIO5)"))
 (segment (start 150.02 87.725942) (end 150.02 92.429744) (width 0.2) (layer "F.Cu") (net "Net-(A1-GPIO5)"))
 (segment (start 150.02 92.429744) (end 150.02 88.110256) (width 0.2) (layer "F.Cu") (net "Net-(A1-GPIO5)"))
 (segment (start 147.285256 87.245) (end 149.539058 87.245) (width 0.2) (layer "F.Cu") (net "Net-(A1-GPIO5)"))
 (segment (start 118.6 94.3) (end 117.5 93.2) (width 0.2) (layer "F.Cu") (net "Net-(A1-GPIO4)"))
 (segment (start 115.602183 95.397817) (end 117.044365 96.84) (width 0.2) (layer "F.Cu") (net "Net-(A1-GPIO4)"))
 (segment (start 117.955635 96.84) (end 118.6 96.195635) (width 0.2) (layer "F.Cu") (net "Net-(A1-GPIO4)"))
 (segment (start 100.95 96.71) (end 102.262183 95.397817) (width 0.2) (layer "F.Cu") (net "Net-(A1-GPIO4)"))
 (segment (start 147.879744 87.795) (end 139.700635 87.795) (width 0.2) (layer "F.Cu") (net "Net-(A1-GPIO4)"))
 (segment (start 100.95 103.53) (end 100.95 96.71) (width 0.2) (layer "F.Cu") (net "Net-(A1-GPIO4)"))
 (segment (start 147.3825 91.745) (end 148.195 90.9325) (width 0.2) (layer "F.Cu") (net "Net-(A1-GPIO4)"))
 (segment (start 148.195 90.9325) (end 148.195 88.110256) (width 0.2) (layer "F.Cu") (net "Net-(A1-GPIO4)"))
 (segment (start 118.6 92.1) (end 117.5 93.2) (width 0.2) (layer "F.Cu") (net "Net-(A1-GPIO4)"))
 (segment (start 102.5 105.08) (end 100.95 103.53) (width 0.2) (layer "F.Cu") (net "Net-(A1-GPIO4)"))
 (segment (start 148.195 88.110256) (end 147.879744 87.795) (width 0.2) (layer "F.Cu") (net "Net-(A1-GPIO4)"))
 (segment (start 135.395635 92.1) (end 118.6 92.1) (width 0.2) (layer "F.Cu") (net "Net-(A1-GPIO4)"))
 (segment (start 117.044365 96.84) (end 117.955635 96.84) (width 0.2) (layer "F.Cu") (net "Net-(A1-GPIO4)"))
 (segment (start 139.700635 87.795) (end 135.395635 92.1) (width 0.2) (layer "F.Cu") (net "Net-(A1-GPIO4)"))
 (segment (start 118.6 96.195635) (end 118.6 94.3) (width 0.2) (layer "F.Cu") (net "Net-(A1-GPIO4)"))
 (segment (start 102.262183 95.397817) (end 115.602183 95.397817) (width 0.2) (layer "F.Cu") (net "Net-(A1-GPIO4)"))
 (segment (start 134.94 91) (end 135.28 90.66) (width 0.2) (layer "F.Cu") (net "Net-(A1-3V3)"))
 (segment (start 148.395 86.529744) (end 148.710256 86.845) (width 0.2) (layer "F.Cu") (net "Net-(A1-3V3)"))
 (segment (start 140.641198 99.5) (end 149.436423 108.295225) (width 0.2) (layer "F.Cu") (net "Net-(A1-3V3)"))
 (segment (start 102.5 97.46) (end 104.54 99.5) (width 0.2) (layer "F.Cu") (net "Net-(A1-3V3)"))
 (segment (start 153.575256 79.98) (end 148.395 85.160256) (width 0.2) (layer "F.Cu") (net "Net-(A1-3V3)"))
 (segment (start 149.436423 108.295225) (end 153.54135 108.295225) (width 0.2) (layer "F.Cu") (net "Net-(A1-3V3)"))
 (segment (start 133 91) (end 134.94 91) (width 0.2) (layer "F.Cu") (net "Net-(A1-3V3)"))
 (segment (start 153.54135 108.295225) (end 154 107.836575) (width 0.2) (layer "F.Cu") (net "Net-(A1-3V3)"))
 (segment (start 150.5 87.640256) (end 150.5 93.4025) (width 0.2) (layer "F.Cu") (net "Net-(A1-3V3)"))
 (segment (start 170.6 80.917258) (end 169.662742 79.98) (width 0.2) (layer "F.Cu") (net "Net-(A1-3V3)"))
 (segment (start 149.2075 91.745) (end 148.074218 92.878282) (width 0.2) (layer "F.Cu") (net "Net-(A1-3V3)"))
 (segment (start 149.704744 86.845) (end 150.5 87.640256) (width 0.2) (layer "F.Cu") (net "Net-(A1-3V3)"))
 (segment (start 150.5 93.4025) (end 149.2075 94.695) (width 0.2) (layer "F.Cu") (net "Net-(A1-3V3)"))
 (segment (start 154 97.517258) (end 168.337258 83.18) (width 0.2) (layer "F.Cu") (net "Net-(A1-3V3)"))
 (segment (start 169.662742 79.98) (end 153.575256 79.98) (width 0.2) (layer "F.Cu") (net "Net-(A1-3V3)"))
 (segment (start 169.662742 83.18) (end 170.6 82.242742) (width 0.2) (layer "F.Cu") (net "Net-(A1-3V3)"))
 (segment (start 148.074218 92.878282) (end 146.8 92.878282) (width 0.2) (layer "F.Cu") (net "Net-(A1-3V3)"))
 (segment (start 128.5 99.5) (end 140.641198 99.5) (width 0.2) (layer "F.Cu") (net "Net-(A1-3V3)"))
 (segment (start 170.6 82.242742) (end 170.6 80.917258) (width 0.2) (layer "F.Cu") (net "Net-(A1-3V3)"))
 (segment (start 148.395 85.160256) (end 148.395 86.529744) (width 0.2) (layer "F.Cu") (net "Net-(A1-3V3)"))
 (segment (start 104.54 99.5) (end 128.5 99.5) (width 0.2) (layer "F.Cu") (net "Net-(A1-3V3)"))
 (segment (start 148.710256 86.845) (end 149.704744 86.845) (width 0.2) (layer "F.Cu") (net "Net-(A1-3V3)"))
 (segment (start 154 107.836575) (end 154 97.517258) (width 0.2) (layer "F.Cu") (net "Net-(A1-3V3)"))
 (segment (start 168.337258 83.18) (end 169.662742 83.18) (width 0.2) (layer "F.Cu") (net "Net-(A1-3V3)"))
 (segment (start 128.5 84.98) (end 128.5 88.96) (width 0.2) (layer "F.Cu") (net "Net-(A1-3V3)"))
 (via (at 133 91) (size 0.6) (drill 0.3) (layers "F.Cu" "B.Cu") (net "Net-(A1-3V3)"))
 (via (at 146.8 92.878282) (size 0.6) (drill 0.3) (layers "F.Cu" "B.Cu") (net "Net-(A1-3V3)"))
 (via (at 128.5 88.96) (size 0.6) (drill 0.3) (layers "F.Cu" "B.Cu") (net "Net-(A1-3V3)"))
 (via (at 128.5 99.5) (size 0.6) (drill 0.3) (layers "F.Cu" "B.Cu") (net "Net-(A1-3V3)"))
 (via (at 128.5 84.98) (size 0.6) (drill 0.3) (layers "F.Cu" "B.Cu") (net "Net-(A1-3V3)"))
 (segment (start 128.5 88.96) (end 128.5 90.5) (width 0.2) (layer "B.Cu") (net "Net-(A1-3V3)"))
 (segment (start 146.8 92.878282) (end 153.9 85.778282) (width 0.2) (layer "B.Cu") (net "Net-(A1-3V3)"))
 (segment (start 153.9 83.834315) (end 153.565685 83.5) (width 0.2) (layer "B.Cu") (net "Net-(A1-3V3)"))
 (segment (start 135.735635 84.14) (end 134.86 84.14) (width 0.2) (layer "B.Cu") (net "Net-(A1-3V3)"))
 (segment (start 134.86 84.14) (end 134.5 84.5) (width 0.2) (layer "B.Cu") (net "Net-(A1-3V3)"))
 (segment (start 128.5 97.44) (end 128.5 99.5) (width 0.2) (layer "B.Cu") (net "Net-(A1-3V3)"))
 (segment (start 134.5 84.5) (end 128.98 84.5) (width 0.2) (layer "B.Cu") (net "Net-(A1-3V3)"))
 (segment (start 128.5 90.5) (end 129 91) (width 0.2) (layer "B.Cu") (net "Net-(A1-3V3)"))
 (segment (start 128.98 84.5) (end 128.5 84.98) (width 0.2) (layer "B.Cu") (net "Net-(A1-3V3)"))
 (segment (start 135.28 90.66) (end 128.5 97.44) (width 0.2) (layer "B.Cu") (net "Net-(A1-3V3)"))
 (segment (start 136.375635 83.5) (end 135.735635 84.14) (width 0.2) (layer "B.Cu") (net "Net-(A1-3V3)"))
 (segment (start 153.565685 83.5) (end 136.375635 83.5) (width 0.2) (layer "B.Cu") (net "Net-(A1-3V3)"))
 (segment (start 153.9 85.778282) (end 153.9 83.834315) (width 0.2) (layer "B.Cu") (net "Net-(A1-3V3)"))
 (segment (start 129 91) (end 133 91) (width 0.2) (layer "B.Cu") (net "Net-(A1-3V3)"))
 (segment (start 105.5 80.58) (end 109.5 84.58) (width 0.2) (layer "F.Cu") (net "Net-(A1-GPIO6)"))
 (segment (start 113 97.5) (end 114 98.5) (width 0.2) (layer "F.Cu") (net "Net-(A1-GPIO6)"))
 (segment (start 115.18 100.82) (end 117.5 100.82) (width 0.2) (layer "F.Cu") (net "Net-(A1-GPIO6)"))
 (segment (start 109.5 84.58) (end 109.5 93) (width 0.2) (layer "F.Cu") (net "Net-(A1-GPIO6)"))
 (segment (start 115 101) (end 115.18 100.82) (width 0.2) (layer "F.Cu") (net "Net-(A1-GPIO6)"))
 (segment (start 110 97.5) (end 113 97.5) (width 0.2) (layer "F.Cu") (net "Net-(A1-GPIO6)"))
 (via (at 109.5 93) (size 0.6) (drill 0.3) (layers "F.Cu" "B.Cu") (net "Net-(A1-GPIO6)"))
 (via (at 110 97.5) (size 0.6) (drill 0.3) (layers "F.Cu" "B.Cu") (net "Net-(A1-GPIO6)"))
 (via (at 114 98.5) (size 0.6) (drill 0.3) (layers "F.Cu" "B.Cu") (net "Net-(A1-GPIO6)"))
 (via (at 115 101) (size 0.6) (drill 0.3) (layers "F.Cu" "B.Cu") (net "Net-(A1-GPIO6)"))
 (segment (start 114 100) (end 115 101) (width 0.2) (layer "B.Cu") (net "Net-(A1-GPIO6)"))
 (segment (start 109.5 93) (end 109.5 97) (width 0.2) (layer "B.Cu") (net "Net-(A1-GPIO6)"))
 (segment (start 114 98.5) (end 114 100) (width 0.2) (layer "B.Cu") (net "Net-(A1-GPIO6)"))
 (segment (start 109.5 97) (end 110 97.5) (width 0.2) (layer "B.Cu") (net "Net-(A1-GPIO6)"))
 (segment (start 111 81) (end 111 93) (width 0.2) (layer "F.Cu") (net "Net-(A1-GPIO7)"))
 (segment (start 115.64 103.36) (end 117.5 103.36) (width 0.2) (layer "F.Cu") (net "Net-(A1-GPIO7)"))
 (segment (start 105.5 75.5) (end 111 81) (width 0.2) (layer "F.Cu") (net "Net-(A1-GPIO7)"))
 (segment (start 115.5 103.5) (end 115.64 103.36) (width 0.2) (layer "F.Cu") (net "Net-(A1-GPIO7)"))
 (via (at 115.5 103.5) (size 0.6) (drill 0.3) (layers "F.Cu" "B.Cu") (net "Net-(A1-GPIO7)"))
 (via (at 111 93) (size 0.6) (drill 0.3) (layers "F.Cu" "B.Cu") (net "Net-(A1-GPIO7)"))
 (segment (start 114 103.5) (end 115.5 103.5) (width 0.2) (layer "B.Cu") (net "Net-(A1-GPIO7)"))
 (segment (start 111 93) (end 111 100.5) (width 0.2) (layer "B.Cu") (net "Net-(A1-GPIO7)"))
 (segment (start 111 100.5) (end 114 103.5) (width 0.2) (layer "B.Cu") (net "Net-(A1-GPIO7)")))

